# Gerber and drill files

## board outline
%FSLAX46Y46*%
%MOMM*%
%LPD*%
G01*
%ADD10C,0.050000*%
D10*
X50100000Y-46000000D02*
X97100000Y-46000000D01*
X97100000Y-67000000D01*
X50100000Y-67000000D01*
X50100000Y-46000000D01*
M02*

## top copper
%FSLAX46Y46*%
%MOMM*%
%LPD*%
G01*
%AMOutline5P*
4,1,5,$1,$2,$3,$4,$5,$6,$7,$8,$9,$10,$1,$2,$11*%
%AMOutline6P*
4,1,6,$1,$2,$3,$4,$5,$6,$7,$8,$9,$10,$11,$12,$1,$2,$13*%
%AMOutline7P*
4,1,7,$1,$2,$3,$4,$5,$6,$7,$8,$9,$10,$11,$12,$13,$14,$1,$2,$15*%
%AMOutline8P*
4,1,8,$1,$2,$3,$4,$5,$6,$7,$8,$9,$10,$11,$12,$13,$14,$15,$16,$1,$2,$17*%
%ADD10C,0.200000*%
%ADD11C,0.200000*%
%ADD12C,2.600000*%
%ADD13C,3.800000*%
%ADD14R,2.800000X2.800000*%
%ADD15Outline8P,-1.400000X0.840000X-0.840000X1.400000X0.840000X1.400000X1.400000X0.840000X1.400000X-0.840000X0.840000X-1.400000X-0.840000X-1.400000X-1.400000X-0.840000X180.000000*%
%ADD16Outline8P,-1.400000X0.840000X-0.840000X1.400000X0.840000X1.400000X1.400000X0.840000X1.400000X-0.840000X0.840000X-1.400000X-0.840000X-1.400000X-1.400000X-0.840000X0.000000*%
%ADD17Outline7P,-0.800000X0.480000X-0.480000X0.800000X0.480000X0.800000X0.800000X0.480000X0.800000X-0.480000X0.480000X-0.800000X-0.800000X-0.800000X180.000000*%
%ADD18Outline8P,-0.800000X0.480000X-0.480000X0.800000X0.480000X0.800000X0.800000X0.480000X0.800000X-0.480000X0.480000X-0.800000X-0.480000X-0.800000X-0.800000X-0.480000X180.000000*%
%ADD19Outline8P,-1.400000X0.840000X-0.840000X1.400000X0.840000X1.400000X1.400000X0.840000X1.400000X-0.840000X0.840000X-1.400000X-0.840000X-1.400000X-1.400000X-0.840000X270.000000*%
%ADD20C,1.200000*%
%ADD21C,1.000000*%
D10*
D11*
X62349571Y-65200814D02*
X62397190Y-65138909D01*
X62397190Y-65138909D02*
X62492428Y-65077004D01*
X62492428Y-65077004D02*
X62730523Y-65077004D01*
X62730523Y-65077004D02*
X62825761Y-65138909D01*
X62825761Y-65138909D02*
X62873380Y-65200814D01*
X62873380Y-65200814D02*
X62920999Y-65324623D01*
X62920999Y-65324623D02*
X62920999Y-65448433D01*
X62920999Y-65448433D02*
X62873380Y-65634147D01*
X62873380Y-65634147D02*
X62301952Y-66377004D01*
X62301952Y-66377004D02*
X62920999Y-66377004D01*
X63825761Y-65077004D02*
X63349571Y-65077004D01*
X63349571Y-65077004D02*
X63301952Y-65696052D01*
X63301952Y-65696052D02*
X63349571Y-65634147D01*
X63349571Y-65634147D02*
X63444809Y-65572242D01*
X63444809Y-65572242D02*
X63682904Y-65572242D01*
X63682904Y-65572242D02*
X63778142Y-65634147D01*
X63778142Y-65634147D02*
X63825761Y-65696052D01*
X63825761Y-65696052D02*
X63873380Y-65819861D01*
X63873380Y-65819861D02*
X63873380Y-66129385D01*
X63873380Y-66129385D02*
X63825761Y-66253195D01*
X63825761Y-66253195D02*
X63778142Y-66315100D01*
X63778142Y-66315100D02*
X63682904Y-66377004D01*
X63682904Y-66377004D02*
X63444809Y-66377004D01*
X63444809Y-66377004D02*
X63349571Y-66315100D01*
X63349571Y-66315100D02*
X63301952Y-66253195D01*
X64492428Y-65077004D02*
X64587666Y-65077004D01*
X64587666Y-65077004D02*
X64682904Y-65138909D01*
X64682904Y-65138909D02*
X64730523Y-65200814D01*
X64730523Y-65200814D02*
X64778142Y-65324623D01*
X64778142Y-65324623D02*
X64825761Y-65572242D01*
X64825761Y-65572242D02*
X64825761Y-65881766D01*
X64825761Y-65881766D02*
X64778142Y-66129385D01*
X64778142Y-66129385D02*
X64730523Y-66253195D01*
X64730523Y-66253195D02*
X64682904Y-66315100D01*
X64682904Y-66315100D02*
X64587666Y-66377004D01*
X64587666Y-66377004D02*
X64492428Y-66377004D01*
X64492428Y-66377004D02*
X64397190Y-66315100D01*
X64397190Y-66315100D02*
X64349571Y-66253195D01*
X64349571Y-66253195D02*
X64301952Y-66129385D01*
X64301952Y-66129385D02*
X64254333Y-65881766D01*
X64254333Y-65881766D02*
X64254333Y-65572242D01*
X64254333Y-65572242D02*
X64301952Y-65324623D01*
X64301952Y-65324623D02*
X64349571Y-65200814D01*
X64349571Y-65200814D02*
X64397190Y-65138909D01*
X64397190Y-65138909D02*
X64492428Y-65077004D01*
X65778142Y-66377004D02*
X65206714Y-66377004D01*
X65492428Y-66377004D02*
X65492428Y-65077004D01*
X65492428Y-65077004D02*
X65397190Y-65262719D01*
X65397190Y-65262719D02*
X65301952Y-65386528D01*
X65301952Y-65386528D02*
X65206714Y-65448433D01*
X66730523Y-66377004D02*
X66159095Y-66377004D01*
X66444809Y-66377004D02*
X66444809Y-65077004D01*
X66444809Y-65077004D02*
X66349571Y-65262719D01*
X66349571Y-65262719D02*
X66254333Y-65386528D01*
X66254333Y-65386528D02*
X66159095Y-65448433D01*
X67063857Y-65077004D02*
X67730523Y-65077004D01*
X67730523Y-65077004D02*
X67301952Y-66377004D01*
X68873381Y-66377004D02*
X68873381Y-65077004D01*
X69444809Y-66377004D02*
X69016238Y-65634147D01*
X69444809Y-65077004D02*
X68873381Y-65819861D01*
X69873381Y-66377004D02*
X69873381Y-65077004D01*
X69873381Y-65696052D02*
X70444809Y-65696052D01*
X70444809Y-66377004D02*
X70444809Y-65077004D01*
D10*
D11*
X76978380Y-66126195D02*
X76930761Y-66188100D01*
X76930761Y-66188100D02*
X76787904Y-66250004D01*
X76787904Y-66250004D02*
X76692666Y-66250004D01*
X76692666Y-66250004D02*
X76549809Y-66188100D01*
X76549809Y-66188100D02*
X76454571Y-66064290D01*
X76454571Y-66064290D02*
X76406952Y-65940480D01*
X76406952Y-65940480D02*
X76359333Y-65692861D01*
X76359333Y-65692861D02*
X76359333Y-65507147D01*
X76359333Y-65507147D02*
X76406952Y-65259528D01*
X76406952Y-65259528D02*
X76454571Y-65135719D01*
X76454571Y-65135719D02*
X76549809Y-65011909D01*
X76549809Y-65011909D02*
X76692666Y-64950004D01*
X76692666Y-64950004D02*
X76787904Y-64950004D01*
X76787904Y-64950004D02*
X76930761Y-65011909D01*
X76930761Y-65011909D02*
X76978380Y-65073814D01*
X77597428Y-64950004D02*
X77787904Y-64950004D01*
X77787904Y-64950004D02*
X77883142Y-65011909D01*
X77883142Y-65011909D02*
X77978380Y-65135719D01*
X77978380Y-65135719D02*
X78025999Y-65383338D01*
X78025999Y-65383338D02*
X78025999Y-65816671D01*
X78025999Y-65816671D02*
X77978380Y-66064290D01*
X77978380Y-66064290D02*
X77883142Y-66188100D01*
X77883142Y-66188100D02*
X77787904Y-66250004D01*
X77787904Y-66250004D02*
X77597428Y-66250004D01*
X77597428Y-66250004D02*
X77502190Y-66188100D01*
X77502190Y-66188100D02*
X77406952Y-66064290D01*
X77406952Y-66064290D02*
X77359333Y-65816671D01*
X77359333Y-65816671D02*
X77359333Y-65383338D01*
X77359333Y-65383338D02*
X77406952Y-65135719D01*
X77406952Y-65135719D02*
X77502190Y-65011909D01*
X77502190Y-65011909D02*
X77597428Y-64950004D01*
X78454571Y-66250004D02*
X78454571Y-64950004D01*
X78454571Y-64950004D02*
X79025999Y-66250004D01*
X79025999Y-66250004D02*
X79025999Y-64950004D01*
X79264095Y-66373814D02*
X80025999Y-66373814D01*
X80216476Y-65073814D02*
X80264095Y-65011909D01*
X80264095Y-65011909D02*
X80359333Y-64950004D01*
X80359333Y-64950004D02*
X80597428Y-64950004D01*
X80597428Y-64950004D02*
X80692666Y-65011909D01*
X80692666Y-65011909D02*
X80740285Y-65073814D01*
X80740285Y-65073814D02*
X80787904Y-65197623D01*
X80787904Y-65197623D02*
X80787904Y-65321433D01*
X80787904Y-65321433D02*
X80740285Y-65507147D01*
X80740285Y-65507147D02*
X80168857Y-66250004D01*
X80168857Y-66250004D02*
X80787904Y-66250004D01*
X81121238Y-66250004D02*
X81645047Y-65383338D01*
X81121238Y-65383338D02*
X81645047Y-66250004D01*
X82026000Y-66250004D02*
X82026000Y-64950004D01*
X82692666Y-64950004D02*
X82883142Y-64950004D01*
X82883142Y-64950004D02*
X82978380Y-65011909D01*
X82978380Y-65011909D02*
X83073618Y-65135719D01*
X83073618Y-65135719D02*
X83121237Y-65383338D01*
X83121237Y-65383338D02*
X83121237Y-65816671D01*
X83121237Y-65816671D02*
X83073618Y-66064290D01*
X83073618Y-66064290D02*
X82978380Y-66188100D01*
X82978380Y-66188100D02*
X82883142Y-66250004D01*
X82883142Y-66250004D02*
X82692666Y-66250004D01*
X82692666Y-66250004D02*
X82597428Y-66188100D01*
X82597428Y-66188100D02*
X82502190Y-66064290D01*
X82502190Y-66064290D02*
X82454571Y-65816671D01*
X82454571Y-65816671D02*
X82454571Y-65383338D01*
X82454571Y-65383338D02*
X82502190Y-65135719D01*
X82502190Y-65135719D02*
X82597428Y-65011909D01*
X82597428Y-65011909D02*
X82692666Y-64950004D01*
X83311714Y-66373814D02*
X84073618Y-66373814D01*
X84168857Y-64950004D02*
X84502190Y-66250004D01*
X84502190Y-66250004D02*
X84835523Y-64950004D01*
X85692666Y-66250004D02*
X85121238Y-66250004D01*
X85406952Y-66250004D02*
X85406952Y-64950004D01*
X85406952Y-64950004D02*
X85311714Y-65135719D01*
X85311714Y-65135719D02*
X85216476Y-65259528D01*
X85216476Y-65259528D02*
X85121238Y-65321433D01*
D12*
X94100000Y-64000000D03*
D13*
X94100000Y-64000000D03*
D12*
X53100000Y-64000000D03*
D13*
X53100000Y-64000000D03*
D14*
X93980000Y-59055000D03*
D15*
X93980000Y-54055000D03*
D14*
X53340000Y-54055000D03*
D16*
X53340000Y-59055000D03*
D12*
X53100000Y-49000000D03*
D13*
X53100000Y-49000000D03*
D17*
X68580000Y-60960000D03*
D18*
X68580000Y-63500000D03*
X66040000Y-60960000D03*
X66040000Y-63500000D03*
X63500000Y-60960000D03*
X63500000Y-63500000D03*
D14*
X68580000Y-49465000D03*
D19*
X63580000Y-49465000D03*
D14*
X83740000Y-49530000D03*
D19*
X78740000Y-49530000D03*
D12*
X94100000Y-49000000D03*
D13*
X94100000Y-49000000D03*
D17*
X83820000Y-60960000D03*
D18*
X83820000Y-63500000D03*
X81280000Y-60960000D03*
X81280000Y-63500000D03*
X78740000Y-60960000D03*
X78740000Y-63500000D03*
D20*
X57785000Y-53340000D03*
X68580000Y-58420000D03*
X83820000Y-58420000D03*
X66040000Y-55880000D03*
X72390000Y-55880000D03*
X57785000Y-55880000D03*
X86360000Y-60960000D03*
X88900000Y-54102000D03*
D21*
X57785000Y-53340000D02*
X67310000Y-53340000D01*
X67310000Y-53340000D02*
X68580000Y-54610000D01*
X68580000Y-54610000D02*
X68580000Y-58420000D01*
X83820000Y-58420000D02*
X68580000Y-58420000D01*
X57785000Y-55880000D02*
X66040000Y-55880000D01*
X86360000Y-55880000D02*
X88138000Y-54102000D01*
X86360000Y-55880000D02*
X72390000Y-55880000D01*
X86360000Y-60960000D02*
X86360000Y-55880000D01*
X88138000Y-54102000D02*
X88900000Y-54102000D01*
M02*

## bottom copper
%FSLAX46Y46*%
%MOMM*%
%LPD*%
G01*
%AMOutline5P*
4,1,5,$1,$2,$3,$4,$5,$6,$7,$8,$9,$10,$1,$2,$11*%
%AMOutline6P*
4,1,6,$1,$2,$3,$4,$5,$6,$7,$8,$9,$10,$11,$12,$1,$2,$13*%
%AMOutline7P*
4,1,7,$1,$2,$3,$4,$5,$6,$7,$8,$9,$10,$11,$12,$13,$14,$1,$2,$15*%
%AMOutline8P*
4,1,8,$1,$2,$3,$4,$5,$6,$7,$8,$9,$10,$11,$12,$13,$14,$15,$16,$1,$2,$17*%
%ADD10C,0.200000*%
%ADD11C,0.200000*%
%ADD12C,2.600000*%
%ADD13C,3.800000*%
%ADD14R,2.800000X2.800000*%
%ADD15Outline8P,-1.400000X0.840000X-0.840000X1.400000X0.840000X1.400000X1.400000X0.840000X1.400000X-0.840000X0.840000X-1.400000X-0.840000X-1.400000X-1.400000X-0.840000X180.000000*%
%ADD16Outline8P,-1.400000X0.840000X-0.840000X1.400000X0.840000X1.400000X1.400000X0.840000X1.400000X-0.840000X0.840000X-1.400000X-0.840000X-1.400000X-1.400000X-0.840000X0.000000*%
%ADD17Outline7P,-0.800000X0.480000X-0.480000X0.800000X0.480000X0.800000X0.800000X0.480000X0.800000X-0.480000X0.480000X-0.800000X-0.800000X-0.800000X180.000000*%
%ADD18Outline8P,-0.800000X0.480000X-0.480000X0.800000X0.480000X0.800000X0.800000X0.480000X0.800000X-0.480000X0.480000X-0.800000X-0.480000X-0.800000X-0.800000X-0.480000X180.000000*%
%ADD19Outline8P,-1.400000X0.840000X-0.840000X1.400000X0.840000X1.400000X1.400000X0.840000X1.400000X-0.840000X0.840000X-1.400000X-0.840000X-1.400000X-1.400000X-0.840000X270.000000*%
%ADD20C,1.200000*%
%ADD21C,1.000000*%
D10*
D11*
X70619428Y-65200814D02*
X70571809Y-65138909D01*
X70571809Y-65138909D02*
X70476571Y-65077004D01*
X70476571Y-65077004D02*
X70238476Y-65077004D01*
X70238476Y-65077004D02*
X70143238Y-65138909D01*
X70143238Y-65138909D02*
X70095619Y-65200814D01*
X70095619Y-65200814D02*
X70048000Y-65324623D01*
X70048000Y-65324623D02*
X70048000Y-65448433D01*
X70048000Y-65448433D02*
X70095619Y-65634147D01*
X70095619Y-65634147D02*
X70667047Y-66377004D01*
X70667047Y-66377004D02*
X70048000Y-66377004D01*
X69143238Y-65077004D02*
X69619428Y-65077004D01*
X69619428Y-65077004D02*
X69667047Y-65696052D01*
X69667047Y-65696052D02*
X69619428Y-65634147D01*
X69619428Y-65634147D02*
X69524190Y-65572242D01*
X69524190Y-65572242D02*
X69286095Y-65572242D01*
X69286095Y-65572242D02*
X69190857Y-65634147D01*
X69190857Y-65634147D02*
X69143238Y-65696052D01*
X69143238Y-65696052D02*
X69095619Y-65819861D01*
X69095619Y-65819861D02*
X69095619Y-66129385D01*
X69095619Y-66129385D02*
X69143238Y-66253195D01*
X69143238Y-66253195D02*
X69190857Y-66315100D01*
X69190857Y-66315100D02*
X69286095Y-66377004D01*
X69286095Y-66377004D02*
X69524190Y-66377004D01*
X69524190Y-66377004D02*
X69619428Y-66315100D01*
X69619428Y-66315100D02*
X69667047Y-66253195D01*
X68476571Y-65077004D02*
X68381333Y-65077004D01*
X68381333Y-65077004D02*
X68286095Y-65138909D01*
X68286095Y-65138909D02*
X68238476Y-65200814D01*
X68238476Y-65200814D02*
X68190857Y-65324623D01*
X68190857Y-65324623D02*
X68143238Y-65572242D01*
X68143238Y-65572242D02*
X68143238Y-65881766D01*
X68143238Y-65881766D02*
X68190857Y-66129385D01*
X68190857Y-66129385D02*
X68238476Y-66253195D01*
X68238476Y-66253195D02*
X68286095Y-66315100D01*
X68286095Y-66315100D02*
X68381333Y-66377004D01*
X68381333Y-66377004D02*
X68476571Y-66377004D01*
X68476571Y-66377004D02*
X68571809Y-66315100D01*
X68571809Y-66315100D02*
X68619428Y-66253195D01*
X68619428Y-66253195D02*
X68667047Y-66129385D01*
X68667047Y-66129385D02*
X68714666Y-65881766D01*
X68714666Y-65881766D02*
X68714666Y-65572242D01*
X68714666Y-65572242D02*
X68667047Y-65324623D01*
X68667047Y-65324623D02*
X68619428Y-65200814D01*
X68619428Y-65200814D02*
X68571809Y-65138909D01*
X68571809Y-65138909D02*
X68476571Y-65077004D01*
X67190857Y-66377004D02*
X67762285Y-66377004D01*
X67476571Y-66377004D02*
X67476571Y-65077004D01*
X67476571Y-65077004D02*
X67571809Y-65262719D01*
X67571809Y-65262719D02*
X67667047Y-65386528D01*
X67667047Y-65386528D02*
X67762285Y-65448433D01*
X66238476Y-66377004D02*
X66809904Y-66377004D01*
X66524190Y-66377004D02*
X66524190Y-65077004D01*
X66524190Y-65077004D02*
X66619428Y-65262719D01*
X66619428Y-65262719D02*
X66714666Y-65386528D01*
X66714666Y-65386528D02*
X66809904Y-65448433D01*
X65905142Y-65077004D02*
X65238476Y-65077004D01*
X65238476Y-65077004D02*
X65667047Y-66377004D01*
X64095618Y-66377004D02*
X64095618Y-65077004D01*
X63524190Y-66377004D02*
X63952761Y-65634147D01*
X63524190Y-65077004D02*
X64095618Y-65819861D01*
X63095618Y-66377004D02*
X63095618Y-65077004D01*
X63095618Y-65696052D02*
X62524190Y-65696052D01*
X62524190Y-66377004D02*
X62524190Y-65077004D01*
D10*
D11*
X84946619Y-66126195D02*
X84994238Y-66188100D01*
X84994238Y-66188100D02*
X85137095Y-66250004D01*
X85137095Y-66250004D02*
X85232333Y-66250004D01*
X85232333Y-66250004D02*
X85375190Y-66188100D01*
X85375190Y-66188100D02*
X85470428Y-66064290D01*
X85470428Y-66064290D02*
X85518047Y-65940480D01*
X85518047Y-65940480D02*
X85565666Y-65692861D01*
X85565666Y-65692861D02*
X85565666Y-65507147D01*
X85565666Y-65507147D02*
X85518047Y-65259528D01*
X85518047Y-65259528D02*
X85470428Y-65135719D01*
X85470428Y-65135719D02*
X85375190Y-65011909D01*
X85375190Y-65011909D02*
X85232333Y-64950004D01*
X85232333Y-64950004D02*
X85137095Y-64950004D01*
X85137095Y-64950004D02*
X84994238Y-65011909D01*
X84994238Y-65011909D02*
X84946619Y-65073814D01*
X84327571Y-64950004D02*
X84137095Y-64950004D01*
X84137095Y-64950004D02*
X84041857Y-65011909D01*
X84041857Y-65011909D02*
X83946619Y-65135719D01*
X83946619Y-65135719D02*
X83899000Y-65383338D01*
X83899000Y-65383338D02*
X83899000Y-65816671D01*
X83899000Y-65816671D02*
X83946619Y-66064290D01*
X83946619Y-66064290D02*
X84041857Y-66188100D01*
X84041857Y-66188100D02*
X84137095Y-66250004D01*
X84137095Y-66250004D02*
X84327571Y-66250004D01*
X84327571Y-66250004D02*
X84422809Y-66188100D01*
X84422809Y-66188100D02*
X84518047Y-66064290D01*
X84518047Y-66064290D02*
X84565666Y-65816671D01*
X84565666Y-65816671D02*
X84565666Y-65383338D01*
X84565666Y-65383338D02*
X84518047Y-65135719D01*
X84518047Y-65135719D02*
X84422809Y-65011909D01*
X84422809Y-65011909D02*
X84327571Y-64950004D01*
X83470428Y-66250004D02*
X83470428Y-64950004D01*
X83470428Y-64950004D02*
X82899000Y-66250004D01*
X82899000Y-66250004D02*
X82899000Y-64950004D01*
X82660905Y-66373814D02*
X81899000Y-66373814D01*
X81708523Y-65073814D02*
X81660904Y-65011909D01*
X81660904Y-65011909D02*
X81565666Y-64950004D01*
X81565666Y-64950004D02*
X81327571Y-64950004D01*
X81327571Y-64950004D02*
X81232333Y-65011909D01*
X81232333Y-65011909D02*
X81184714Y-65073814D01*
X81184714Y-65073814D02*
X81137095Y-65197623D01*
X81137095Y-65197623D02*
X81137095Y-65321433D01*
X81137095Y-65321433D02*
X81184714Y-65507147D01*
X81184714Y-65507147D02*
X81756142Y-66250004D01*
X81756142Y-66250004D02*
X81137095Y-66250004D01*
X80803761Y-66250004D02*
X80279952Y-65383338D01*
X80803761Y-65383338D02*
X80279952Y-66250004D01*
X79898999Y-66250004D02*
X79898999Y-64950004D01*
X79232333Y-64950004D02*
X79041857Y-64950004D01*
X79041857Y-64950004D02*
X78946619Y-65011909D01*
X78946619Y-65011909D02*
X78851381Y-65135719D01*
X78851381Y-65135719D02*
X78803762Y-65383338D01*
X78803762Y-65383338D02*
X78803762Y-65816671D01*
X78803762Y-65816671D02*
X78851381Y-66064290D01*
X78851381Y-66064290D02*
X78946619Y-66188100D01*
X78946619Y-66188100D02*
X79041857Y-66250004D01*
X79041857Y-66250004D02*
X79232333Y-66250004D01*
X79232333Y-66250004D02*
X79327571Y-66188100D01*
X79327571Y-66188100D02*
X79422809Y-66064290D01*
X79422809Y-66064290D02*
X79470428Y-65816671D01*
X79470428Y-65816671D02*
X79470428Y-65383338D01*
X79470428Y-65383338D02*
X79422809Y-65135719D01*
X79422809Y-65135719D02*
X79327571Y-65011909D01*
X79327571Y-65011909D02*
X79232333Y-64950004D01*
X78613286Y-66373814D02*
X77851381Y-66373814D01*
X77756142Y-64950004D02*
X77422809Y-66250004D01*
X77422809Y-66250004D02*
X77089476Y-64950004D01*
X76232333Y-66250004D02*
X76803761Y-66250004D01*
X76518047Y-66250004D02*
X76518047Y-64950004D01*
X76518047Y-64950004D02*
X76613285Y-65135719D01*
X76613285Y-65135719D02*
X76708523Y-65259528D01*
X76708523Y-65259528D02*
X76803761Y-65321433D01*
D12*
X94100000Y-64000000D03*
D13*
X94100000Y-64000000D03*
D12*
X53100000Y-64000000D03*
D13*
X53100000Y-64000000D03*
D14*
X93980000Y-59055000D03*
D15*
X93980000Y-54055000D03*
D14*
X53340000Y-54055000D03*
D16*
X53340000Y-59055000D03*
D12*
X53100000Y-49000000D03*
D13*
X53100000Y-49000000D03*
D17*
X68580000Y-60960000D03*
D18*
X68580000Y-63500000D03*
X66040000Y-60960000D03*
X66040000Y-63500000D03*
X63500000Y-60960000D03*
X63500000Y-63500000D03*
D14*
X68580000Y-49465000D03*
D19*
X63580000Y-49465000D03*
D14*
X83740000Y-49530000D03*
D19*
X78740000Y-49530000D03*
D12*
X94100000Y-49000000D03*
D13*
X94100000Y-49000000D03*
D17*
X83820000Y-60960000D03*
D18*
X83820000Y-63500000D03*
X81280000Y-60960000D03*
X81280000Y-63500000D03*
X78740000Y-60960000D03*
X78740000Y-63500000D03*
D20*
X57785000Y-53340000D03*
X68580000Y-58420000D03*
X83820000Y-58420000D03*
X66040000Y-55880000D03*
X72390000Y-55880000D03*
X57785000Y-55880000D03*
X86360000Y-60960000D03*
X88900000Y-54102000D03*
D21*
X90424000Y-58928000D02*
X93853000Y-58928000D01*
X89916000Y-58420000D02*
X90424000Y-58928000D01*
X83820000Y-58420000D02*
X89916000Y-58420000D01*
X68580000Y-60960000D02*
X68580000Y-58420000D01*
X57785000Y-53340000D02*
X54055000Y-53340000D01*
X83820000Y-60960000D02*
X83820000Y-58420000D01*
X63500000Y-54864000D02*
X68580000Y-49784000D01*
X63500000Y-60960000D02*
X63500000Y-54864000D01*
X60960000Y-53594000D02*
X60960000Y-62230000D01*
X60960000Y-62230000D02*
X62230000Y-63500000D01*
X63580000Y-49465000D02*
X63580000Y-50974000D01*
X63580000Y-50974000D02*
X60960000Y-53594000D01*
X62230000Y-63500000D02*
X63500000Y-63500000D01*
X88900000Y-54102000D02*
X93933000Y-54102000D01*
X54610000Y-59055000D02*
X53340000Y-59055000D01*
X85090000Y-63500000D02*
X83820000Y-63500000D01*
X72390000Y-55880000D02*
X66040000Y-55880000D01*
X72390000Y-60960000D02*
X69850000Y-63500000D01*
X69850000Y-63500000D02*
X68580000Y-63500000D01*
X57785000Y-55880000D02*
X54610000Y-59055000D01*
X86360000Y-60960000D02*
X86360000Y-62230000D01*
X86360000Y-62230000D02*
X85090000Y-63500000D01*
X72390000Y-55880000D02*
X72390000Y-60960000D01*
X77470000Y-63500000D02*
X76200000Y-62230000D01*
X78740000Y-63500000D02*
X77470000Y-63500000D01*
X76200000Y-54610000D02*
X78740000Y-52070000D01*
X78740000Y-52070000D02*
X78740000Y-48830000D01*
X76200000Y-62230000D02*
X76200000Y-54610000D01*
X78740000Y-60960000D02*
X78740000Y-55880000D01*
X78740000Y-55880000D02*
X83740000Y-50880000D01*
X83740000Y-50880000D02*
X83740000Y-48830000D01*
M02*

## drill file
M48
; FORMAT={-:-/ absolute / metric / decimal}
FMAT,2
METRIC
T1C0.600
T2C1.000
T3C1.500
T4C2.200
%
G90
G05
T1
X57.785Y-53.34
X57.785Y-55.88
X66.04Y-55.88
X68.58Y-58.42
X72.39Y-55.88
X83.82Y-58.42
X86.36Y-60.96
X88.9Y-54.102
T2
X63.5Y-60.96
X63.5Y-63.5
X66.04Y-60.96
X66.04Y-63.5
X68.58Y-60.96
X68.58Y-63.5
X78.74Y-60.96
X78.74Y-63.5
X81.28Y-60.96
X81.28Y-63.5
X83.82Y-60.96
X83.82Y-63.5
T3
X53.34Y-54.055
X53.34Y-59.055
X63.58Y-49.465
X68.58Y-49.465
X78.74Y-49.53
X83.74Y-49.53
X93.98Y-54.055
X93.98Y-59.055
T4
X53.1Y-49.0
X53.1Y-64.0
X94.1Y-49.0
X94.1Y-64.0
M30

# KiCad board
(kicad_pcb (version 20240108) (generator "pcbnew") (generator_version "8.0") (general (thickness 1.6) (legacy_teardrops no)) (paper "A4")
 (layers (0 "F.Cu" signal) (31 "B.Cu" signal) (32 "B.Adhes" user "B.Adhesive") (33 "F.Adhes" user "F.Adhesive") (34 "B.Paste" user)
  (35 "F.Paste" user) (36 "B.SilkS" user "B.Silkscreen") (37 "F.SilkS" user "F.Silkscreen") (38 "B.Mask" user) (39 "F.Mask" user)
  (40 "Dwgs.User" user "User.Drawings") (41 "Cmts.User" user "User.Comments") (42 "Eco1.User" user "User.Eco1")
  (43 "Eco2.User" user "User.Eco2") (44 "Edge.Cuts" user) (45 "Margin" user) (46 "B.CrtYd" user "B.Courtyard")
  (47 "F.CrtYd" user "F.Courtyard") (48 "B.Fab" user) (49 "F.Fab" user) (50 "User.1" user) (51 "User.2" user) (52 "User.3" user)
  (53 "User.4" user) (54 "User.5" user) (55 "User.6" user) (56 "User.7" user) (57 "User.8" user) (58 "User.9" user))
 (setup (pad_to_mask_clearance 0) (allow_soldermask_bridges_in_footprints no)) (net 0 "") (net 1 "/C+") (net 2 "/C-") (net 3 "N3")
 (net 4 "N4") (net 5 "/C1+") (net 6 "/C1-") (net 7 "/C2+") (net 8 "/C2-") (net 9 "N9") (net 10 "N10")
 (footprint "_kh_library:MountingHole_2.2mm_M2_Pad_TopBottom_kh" (layer "F.Cu") (at 94.1 64)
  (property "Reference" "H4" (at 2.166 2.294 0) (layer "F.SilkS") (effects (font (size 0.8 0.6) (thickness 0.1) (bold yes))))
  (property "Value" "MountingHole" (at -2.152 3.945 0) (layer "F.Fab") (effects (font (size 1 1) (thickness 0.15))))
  (pad "1" thru_hole circle (at 0 0) (size 2.6 2.6) (drill 2.2) (layers "*.Cu" "*.Mask") (remove_unused_layers no))
  (pad "1" connect circle (at 0 0) (size 3.8 3.8) (layers "F.Cu" "F.Mask"))
  (pad "1" connect circle (at 0 0) (size 3.8 3.8) (layers "B.Cu" "B.Mask")))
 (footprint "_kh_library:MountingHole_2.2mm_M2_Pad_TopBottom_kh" (layer "F.Cu") (at 53.1 64)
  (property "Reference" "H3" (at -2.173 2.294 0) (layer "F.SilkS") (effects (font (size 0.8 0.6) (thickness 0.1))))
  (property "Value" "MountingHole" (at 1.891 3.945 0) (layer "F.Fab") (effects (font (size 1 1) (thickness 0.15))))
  (pad "1" thru_hole circle (at 0 0) (size 2.6 2.6) (drill 2.2) (layers "*.Cu" "*.Mask") (remove_unused_layers no))
  (pad "1" connect circle (at 0 0) (size 3.8 3.8) (layers "F.Cu" "F.Mask"))
  (pad "1" connect circle (at 0 0) (size 3.8 3.8) (layers "B.Cu" "B.Mask")))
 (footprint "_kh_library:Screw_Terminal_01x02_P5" (layer "F.Cu") (at 93.98 59.055 180)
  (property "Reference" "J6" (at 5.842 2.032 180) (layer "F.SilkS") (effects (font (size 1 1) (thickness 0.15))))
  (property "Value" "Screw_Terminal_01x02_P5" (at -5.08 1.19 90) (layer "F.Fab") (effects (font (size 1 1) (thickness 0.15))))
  (pad "1" thru_hole rect (at 0 0 180) (size 2.8 2.8) (drill 1.5) (layers "*.Cu" "*.Mask") (remove_unused_layers no) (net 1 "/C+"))
  (pad "2" thru_hole roundrect (at 0 5 180) (size 2.8 2.8) (drill 1.5) (layers "*.Cu" "*.Mask") (remove_unused_layers no)
   (roundrect_rratio 0) (chamfer_ratio 0.2) (chamfer top_left top_right bottom_left bottom_right) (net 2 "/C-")))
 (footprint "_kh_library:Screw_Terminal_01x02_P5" (layer "F.Cu") (at 53.34 54.055)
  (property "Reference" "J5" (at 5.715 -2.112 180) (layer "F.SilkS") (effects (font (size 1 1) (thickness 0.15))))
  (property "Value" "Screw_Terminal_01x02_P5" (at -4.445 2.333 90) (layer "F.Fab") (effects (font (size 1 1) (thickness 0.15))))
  (pad "1" thru_hole rect (at 0 0) (size 2.8 2.8) (drill 1.5) (layers "*.Cu" "*.Mask") (remove_unused_layers no) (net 1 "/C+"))
  (pad "2" thru_hole roundrect (at 0 5) (size 2.8 2.8) (drill 1.5) (layers "*.Cu" "*.Mask") (remove_unused_layers no) (roundrect_rratio 0)
   (chamfer_ratio 0.2) (chamfer top_left top_right bottom_left bottom_right) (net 2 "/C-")))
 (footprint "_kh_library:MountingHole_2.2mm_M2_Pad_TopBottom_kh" (layer "F.Cu") (at 53.1 49)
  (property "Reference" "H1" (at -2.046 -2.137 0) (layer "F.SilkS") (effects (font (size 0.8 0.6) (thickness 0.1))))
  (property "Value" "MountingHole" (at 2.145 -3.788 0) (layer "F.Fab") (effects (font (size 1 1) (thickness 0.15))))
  (pad "1" thru_hole circle (at 0 0) (size 2.6 2.6) (drill 2.2) (layers "*.Cu" "*.Mask") (remove_unused_layers no))
  (pad "1" connect circle (at 0 0) (size 3.8 3.8) (layers "F.Cu" "F.Mask"))
  (pad "1" connect circle (at 0 0) (size 3.8 3.8) (layers "B.Cu" "B.Mask")))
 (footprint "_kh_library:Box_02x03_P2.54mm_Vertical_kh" (layer "F.Cu") (at 68.58 60.96 180)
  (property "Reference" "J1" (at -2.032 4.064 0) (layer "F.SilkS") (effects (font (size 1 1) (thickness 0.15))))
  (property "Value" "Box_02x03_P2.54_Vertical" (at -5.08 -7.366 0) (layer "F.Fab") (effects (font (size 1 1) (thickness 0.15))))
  (pad "1" thru_hole roundrect (at 0 0 180) (size 1.6 1.6) (drill 1) (layers "*.Cu" "*.Mask") (remove_unused_layers no) (roundrect_rratio 0)
   (chamfer_ratio 0.2) (chamfer top_left top_right bottom_right) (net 1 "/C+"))
  (pad "2" thru_hole roundrect (at 0 -2.54 180) (size 1.6 1.6) (drill 1) (layers "*.Cu" "*.Mask") (remove_unused_layers no)
   (roundrect_rratio 0) (chamfer_ratio 0.2) (chamfer top_left top_right bottom_left bottom_right) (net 2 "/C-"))
  (pad "3" thru_hole roundrect (at 2.54 0 180) (size 1.6 1.6) (drill 1) (layers "*.Cu" "*.Mask") (remove_unused_layers no)
   (roundrect_rratio 0) (chamfer_ratio 0.2) (chamfer top_left top_right bottom_left bottom_right) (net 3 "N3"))
  (pad "4" thru_hole roundrect (at 2.54 -2.54 180) (size 1.6 1.6) (drill 1) (layers "*.Cu" "*.Mask") (remove_unused_layers no)
   (roundrect_rratio 0) (chamfer_ratio 0.2) (chamfer top_left top_right bottom_left bottom_right) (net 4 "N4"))
  (pad "5" thru_hole roundrect (at 5.08 0 180) (size 1.6 1.6) (drill 1) (layers "*.Cu" "*.Mask") (remove_unused_layers no)
   (roundrect_rratio 0) (chamfer_ratio 0.2) (chamfer top_left top_right bottom_left bottom_right) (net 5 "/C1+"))
  (pad "6" thru_hole roundrect (at 5.08 -2.54 180) (size 1.6 1.6) (drill 1) (layers "*.Cu" "*.Mask") (remove_unused_layers no)
   (roundrect_rratio 0) (chamfer_ratio 0.2) (chamfer top_left top_right bottom_left bottom_right) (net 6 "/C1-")))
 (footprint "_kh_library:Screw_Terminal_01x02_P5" (layer "F.Cu") (at 68.58 49.465 -90)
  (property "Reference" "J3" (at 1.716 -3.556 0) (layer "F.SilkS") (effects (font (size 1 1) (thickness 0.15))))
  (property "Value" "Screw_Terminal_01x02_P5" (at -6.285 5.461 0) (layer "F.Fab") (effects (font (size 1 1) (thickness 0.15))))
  (pad "1" thru_hole rect (at 0 0 270) (size 2.8 2.8) (drill 1.5) (layers "*.Cu" "*.Mask") (remove_unused_layers no) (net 5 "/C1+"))
  (pad "2" thru_hole roundrect (at 0 5 270) (size 2.8 2.8) (drill 1.5) (layers "*.Cu" "*.Mask") (remove_unused_layers no)
   (roundrect_rratio 0) (chamfer_ratio 0.2) (chamfer top_left top_right bottom_left bottom_right) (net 6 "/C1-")))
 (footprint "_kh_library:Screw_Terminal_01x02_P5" (layer "F.Cu") (at 83.74 49.53 -90)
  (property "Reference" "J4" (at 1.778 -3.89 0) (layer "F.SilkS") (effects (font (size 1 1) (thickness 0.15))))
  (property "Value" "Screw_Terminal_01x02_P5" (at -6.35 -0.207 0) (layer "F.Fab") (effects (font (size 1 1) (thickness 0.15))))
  (pad "1" thru_hole rect (at 0 0 270) (size 2.8 2.8) (drill 1.5) (layers "*.Cu" "*.Mask") (remove_unused_layers no) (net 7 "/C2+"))
  (pad "2" thru_hole roundrect (at 0 5 270) (size 2.8 2.8) (drill 1.5) (layers "*.Cu" "*.Mask") (remove_unused_layers no)
   (roundrect_rratio 0) (chamfer_ratio 0.2) (chamfer top_left top_right bottom_left bottom_right) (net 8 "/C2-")))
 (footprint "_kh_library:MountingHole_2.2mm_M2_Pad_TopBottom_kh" (layer "F.Cu") (at 94.1 49)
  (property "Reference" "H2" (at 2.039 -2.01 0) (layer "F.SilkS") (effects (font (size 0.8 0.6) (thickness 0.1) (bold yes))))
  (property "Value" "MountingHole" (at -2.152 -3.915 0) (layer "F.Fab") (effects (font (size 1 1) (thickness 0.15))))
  (pad "1" thru_hole circle (at 0 0) (size 2.6 2.6) (drill 2.2) (layers "*.Cu" "*.Mask") (remove_unused_layers no))
  (pad "1" connect circle (at 0 0) (size 3.8 3.8) (layers "F.Cu" "F.Mask"))
  (pad "1" connect circle (at 0 0) (size 3.8 3.8) (layers "B.Cu" "B.Mask")))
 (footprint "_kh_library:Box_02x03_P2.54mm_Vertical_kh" (layer "F.Cu") (at 83.82 60.96 180)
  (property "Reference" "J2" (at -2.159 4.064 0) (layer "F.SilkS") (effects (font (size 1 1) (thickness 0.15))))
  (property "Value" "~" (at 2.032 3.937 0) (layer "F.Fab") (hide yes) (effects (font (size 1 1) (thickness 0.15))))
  (pad "1" thru_hole roundrect (at 0 0 180) (size 1.6 1.6) (drill 1) (layers "*.Cu" "*.Mask") (remove_unused_layers no) (roundrect_rratio 0)
   (chamfer_ratio 0.2) (chamfer top_left top_right bottom_right) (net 1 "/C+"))
  (pad "2" thru_hole roundrect (at 0 -2.54 180) (size 1.6 1.6) (drill 1) (layers "*.Cu" "*.Mask") (remove_unused_layers no)
   (roundrect_rratio 0) (chamfer_ratio 0.2) (chamfer top_left top_right bottom_left bottom_right) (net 2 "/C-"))
  (pad "3" thru_hole roundrect (at 2.54 0 180) (size 1.6 1.6) (drill 1) (layers "*.Cu" "*.Mask") (remove_unused_layers no)
   (roundrect_rratio 0) (chamfer_ratio 0.2) (chamfer top_left top_right bottom_left bottom_right) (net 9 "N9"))
  (pad "4" thru_hole roundrect (at 2.54 -2.54 180) (size 1.6 1.6) (drill 1) (layers "*.Cu" "*.Mask") (remove_unused_layers no)
   (roundrect_rratio 0) (chamfer_ratio 0.2) (chamfer top_left top_right bottom_left bottom_right) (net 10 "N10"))
  (pad "5" thru_hole roundrect (at 5.08 0 180) (size 1.6 1.6) (drill 1) (layers "*.Cu" "*.Mask") (remove_unused_layers no)
   (roundrect_rratio 0) (chamfer_ratio 0.2) (chamfer top_left top_right bottom_left bottom_right) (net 7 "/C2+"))
  (pad "6" thru_hole roundrect (at 5.08 -2.54 180) (size 1.6 1.6) (drill 1) (layers "*.Cu" "*.Mask") (remove_unused_layers no)
   (roundrect_rratio 0) (chamfer_ratio 0.2) (chamfer top_left top_right bottom_left bottom_right) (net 8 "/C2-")))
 (gr_rect (start 50.1 46) (end 97.1 67) (stroke (width 0.05) (type default)) (fill none) (layer "Edge.Cuts"))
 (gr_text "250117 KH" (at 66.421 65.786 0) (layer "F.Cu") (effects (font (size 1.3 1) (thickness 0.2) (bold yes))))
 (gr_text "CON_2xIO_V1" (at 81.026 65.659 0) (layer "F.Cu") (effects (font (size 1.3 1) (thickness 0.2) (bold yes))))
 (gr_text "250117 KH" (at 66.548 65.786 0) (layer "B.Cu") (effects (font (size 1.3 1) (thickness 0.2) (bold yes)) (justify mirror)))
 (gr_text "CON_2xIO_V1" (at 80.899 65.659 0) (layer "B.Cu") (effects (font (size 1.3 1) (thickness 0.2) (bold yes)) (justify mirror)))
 (segment (start 57.785 53.34) (end 67.31 53.34) (width 1) (layer "F.Cu") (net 1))
 (segment (start 67.31 53.34) (end 68.58 54.61) (width 1) (layer "F.Cu") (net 1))
 (segment (start 68.58 54.61) (end 68.58 58.42) (width 1) (layer "F.Cu") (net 1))
 (segment (start 83.82 58.42) (end 68.58 58.42) (width 1) (layer "F.Cu") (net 1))
 (via (at 57.785 53.34) (size 1.2) (drill 0.6) (layers "F.Cu" "B.Cu") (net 1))
 (via (at 68.58 58.42) (size 1.2) (drill 0.6) (layers "F.Cu" "B.Cu") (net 1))
 (via (at 83.82 58.42) (size 1.2) (drill 0.6) (layers "F.Cu" "B.Cu") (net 1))
 (segment (start 90.424 58.928) (end 93.853 58.928) (width 1) (layer "B.Cu") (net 1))
 (segment (start 89.916 58.42) (end 90.424 58.928) (width 1) (layer "B.Cu") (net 1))
 (segment (start 83.82 58.42) (end 89.916 58.42) (width 1) (layer "B.Cu") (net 1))
 (segment (start 68.58 60.96) (end 68.58 58.42) (width 1) (layer "B.Cu") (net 1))
 (segment (start 57.785 53.34) (end 54.055 53.34) (width 1) (layer "B.Cu") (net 1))
 (segment (start 83.82 60.96) (end 83.82 58.42) (width 1) (layer "B.Cu") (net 1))
 (segment (start 63.5 54.864) (end 68.58 49.784) (width 1) (layer "B.Cu") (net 5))
 (segment (start 63.5 60.96) (end 63.5 54.864) (width 1) (layer "B.Cu") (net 5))
 (segment (start 60.96 53.594) (end 60.96 62.23) (width 1) (layer "B.Cu") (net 6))
 (segment (start 60.96 62.23) (end 62.23 63.5) (width 1) (layer "B.Cu") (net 6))
 (segment (start 63.58 49.465) (end 63.58 50.974) (width 1) (layer "B.Cu") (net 6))
 (segment (start 63.58 50.974) (end 60.96 53.594) (width 1) (layer "B.Cu") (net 6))
 (segment (start 62.23 63.5) (end 63.5 63.5) (width 1) (layer "B.Cu") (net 6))
 (segment (start 57.785 55.88) (end 66.04 55.88) (width 1) (layer "F.Cu") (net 2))
 (segment (start 86.36 55.88) (end 88.138 54.102) (width 1) (layer "F.Cu") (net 2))
 (segment (start 86.36 55.88) (end 72.39 55.88) (width 1) (layer "F.Cu") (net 2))
 (segment (start 86.36 60.96) (end 86.36 55.88) (width 1) (layer "F.Cu") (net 2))
 (segment (start 88.138 54.102) (end 88.9 54.102) (width 1) (layer "F.Cu") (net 2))
 (via (at 66.04 55.88) (size 1.2) (drill 0.6) (layers "F.Cu" "B.Cu") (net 2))
 (via (at 72.39 55.88) (size 1.2) (drill 0.6) (layers "F.Cu" "B.Cu") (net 2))
 (via (at 57.785 55.88) (size 1.2) (drill 0.6) (layers "F.Cu" "B.Cu") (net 2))
 (via (at 86.36 60.96) (size 1.2) (drill 0.6) (layers "F.Cu" "B.Cu") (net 2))
 (via (at 88.9 54.102) (size 1.2) (drill 0.6) (layers "F.Cu" "B.Cu") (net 2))
 (segment (start 88.9 54.102) (end 93.933 54.102) (width 1) (layer "B.Cu") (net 2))
 (segment (start 54.61 59.055) (end 53.34 59.055) (width 1) (layer "B.Cu") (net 2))
 (segment (start 85.09 63.5) (end 83.82 63.5) (width 1) (layer "B.Cu") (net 2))
 (segment (start 72.39 55.88) (end 66.04 55.88) (width 1) (layer "B.Cu") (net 2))
 (segment (start 72.39 60.96) (end 69.85 63.5) (width 1) (layer "B.Cu") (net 2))
 (segment (start 69.85 63.5) (end 68.58 63.5) (width 1) (layer "B.Cu") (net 2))
 (segment (start 57.785 55.88) (end 54.61 59.055) (width 1) (layer "B.Cu") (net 2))
 (segment (start 86.36 60.96) (end 86.36 62.23) (width 1) (layer "B.Cu") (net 2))
 (segment (start 86.36 62.23) (end 85.09 63.5) (width 1) (layer "B.Cu") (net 2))
 (segment (start 72.39 55.88) (end 72.39 60.96) (width 1) (layer "B.Cu") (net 2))
 (segment (start 77.47 63.5) (end 76.2 62.23) (width 1) (layer "B.Cu") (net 8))
 (segment (start 78.74 63.5) (end 77.47 63.5) (width 1) (layer "B.Cu") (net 8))
 (segment (start 76.2 54.61) (end 78.74 52.07) (width 1) (layer "B.Cu") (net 8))
 (segment (start 78.74 52.07) (end 78.74 48.83) (width 1) (layer "B.Cu") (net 8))
 (segment (start 76.2 62.23) (end 76.2 54.61) (width 1) (layer "B.Cu") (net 8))
 (segment (start 78.74 60.96) (end 78.74 55.88) (width 1) (layer "B.Cu") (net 7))
 (segment (start 78.74 55.88) (end 83.74 50.88) (width 1) (layer "B.Cu") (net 7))
 (segment (start 83.74 50.88) (end 83.74 48.83) (width 1) (layer "B.Cu") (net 7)))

